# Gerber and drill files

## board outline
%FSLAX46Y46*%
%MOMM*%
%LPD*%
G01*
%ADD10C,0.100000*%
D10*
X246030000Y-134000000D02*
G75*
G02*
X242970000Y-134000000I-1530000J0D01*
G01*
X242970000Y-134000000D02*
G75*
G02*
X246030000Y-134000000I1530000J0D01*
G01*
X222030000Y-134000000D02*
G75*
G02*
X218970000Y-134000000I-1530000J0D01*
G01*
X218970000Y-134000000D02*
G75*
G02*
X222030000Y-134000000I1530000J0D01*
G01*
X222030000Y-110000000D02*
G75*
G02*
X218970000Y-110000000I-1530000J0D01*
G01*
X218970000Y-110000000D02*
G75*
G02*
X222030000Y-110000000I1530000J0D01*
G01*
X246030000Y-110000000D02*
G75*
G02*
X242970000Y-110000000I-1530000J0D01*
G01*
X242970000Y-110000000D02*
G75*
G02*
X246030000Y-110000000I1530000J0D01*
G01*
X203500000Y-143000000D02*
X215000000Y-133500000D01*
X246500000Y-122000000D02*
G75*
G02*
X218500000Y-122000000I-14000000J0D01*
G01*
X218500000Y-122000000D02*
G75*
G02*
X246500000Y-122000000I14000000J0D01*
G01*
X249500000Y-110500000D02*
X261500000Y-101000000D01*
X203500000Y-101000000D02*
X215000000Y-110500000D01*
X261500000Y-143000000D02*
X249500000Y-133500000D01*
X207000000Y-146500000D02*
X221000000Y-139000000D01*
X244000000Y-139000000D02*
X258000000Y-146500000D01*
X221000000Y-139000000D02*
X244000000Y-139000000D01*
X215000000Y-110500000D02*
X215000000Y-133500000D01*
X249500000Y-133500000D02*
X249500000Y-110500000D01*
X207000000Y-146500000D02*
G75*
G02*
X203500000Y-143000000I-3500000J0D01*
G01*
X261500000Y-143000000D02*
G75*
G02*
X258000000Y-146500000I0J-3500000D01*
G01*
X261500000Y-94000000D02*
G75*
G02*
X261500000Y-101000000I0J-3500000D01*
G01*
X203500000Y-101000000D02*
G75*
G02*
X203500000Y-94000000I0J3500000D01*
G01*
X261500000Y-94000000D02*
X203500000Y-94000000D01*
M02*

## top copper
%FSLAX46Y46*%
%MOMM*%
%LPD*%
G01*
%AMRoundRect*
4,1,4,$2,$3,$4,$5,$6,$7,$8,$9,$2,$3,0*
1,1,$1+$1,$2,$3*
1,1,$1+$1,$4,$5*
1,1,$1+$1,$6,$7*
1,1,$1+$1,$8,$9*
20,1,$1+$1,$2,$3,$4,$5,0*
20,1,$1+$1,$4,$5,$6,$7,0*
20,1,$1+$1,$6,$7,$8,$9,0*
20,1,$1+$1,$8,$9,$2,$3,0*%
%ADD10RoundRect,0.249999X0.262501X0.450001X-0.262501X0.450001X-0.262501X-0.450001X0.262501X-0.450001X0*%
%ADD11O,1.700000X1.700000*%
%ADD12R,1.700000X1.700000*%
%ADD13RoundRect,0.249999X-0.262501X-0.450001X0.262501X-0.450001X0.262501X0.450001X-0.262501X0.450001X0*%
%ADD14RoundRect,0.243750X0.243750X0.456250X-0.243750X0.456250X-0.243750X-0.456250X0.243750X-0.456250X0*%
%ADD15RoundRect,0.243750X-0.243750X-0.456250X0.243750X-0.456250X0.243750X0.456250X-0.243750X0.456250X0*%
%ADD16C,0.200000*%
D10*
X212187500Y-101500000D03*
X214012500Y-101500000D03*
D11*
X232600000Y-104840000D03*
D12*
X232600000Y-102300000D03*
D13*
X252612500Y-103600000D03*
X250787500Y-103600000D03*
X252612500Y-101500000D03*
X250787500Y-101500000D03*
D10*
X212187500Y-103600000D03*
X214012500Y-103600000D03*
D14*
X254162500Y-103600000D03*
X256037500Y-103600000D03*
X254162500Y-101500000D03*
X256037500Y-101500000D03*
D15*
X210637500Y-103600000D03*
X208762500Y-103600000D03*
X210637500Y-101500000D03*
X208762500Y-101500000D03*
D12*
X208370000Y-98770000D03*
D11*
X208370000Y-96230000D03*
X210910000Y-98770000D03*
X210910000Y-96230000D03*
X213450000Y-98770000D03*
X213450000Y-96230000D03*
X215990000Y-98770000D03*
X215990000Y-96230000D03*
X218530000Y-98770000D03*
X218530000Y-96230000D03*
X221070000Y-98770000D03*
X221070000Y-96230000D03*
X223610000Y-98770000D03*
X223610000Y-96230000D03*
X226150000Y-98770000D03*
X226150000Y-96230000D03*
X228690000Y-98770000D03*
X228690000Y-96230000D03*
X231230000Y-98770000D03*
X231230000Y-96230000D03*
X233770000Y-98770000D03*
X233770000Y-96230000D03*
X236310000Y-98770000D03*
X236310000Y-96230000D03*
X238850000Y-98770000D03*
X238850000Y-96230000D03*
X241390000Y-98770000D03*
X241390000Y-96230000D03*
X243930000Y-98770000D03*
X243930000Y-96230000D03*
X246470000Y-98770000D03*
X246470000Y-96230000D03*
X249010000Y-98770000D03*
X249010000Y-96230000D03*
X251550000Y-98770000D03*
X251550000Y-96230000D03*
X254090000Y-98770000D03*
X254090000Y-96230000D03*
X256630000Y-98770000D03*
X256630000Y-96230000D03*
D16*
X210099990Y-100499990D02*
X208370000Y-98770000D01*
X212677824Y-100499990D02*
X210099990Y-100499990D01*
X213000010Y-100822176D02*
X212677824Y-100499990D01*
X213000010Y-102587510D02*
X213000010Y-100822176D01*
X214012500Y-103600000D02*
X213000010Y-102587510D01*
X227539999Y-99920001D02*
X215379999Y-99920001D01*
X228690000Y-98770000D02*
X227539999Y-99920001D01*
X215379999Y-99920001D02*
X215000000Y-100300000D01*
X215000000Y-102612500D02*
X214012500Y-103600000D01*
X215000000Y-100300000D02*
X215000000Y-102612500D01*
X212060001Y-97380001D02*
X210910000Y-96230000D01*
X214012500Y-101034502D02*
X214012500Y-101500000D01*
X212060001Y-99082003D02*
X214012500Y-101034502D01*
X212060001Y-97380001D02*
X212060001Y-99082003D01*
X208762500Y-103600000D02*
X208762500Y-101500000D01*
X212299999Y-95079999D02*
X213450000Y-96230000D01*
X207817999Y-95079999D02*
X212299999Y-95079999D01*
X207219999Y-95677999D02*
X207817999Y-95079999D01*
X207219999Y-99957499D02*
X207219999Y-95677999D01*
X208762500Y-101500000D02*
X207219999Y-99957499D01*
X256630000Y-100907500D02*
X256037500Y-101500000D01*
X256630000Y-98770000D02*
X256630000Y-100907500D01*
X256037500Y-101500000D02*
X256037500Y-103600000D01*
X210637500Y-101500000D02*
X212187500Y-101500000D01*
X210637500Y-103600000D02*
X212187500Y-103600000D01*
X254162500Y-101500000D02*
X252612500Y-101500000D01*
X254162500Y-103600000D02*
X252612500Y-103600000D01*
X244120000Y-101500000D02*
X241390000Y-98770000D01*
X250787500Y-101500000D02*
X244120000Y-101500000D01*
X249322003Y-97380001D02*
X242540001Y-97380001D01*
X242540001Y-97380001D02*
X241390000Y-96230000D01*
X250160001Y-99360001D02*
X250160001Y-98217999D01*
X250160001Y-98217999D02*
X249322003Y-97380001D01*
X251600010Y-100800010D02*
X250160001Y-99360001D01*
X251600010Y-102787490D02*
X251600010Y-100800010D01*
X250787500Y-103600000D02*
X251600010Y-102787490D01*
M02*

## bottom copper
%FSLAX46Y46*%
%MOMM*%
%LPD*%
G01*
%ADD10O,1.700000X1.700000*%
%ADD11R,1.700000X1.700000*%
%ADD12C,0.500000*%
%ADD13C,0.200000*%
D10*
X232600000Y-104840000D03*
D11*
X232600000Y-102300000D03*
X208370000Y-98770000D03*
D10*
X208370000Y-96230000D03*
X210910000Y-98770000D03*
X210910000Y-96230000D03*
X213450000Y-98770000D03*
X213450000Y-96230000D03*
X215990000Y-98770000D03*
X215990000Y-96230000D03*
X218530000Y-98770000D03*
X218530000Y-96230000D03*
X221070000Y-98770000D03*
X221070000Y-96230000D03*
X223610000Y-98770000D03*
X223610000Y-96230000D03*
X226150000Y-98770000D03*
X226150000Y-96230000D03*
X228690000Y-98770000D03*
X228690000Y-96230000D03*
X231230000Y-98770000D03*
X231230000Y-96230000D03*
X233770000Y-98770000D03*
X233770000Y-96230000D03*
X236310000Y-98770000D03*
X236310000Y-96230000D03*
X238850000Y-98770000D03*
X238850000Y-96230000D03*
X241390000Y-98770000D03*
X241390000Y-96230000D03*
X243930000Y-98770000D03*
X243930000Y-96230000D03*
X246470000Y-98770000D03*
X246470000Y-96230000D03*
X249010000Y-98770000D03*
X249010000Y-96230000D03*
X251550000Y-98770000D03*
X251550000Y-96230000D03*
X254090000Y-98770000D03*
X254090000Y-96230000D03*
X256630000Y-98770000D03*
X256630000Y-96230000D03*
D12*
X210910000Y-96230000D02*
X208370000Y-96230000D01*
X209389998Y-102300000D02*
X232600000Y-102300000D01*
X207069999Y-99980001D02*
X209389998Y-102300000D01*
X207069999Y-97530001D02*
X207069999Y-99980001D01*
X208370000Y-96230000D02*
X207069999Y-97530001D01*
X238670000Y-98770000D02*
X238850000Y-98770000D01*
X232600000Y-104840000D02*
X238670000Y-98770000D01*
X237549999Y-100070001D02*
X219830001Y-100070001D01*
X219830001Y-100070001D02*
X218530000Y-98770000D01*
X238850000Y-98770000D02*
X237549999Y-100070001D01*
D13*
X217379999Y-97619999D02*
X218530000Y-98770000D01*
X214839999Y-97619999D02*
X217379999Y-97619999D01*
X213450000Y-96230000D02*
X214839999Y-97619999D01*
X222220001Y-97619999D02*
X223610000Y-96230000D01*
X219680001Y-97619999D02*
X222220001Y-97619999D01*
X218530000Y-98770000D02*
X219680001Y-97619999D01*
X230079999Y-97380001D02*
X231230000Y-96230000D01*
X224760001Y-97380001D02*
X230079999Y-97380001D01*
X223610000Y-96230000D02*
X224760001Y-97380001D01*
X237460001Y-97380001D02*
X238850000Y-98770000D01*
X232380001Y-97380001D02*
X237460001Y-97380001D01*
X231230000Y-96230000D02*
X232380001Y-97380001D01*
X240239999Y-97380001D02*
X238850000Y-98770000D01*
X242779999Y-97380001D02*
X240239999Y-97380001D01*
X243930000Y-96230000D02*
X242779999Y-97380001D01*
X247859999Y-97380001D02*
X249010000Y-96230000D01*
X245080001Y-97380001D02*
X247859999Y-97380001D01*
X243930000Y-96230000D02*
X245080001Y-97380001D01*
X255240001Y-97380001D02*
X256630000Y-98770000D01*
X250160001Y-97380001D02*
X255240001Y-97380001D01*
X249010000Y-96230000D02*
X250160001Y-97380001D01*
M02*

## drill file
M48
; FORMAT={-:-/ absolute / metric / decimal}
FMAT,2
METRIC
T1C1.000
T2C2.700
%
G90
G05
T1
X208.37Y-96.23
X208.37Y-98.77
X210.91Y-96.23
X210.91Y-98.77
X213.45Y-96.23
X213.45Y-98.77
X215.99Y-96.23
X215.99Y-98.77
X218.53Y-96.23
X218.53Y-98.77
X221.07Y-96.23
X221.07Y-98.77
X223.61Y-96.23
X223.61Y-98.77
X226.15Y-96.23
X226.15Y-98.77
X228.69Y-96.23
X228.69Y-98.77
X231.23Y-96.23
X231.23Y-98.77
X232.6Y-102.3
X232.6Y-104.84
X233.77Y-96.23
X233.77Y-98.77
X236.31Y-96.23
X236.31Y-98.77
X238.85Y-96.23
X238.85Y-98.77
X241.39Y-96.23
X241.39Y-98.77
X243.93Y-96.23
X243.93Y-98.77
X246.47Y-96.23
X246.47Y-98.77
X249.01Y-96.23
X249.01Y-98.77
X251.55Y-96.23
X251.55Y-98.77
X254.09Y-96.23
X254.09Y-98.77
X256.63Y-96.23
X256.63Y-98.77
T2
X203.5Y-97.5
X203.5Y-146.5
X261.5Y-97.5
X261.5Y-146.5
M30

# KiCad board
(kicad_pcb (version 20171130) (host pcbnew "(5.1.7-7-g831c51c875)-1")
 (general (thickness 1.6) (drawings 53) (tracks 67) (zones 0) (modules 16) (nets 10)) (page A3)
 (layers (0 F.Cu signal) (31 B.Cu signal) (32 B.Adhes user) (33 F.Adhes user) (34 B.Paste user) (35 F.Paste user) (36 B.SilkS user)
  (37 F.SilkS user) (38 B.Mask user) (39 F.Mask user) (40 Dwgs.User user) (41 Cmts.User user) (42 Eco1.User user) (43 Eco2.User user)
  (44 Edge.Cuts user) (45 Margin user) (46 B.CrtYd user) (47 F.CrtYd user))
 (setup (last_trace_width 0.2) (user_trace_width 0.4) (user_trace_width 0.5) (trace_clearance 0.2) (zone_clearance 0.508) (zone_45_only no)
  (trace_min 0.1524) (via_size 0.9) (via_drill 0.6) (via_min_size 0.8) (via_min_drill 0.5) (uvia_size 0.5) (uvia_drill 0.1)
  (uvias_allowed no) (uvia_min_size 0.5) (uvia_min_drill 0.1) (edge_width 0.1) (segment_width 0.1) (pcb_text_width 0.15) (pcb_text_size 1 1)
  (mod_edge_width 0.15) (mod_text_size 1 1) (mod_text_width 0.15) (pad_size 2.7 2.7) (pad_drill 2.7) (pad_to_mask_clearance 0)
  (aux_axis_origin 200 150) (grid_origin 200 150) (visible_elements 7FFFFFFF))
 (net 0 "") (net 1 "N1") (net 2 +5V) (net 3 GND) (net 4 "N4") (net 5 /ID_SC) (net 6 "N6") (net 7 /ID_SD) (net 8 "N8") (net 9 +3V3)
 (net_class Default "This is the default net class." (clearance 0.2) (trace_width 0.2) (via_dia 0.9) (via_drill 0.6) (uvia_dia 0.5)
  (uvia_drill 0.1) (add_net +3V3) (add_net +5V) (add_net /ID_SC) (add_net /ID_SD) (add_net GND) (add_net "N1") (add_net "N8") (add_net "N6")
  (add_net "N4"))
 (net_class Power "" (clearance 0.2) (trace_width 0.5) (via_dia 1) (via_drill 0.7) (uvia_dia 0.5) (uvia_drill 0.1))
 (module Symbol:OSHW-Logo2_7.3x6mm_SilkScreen (layer F.Cu) (at 251 138.3)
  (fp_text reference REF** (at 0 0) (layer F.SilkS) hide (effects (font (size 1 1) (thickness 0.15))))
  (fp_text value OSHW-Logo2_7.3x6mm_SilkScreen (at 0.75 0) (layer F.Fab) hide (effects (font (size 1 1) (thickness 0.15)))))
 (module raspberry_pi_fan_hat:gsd (layer F.Cu) (at 213.9 138.30663)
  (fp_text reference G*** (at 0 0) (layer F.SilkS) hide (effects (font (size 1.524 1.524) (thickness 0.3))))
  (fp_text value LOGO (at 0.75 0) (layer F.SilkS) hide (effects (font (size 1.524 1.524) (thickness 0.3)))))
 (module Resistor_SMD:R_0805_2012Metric (layer F.Cu) (at 213.1 101.5 180)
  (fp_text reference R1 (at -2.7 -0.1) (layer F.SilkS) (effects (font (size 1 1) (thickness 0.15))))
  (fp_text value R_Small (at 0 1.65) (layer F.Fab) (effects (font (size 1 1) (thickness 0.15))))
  (pad 2 smd roundrect (at 0.9125 0 180) (size 1.025 1.4) (layers F.Cu F.Paste F.Mask) (roundrect_rratio 0.2439014634146341) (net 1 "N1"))
  (pad 1 smd roundrect (at -0.9125 0 180) (size 1.025 1.4) (layers F.Cu F.Paste F.Mask) (roundrect_rratio 0.2439014634146341) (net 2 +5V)))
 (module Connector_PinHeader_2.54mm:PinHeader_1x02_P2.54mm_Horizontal (layer F.Cu) (at 232.6 102.3)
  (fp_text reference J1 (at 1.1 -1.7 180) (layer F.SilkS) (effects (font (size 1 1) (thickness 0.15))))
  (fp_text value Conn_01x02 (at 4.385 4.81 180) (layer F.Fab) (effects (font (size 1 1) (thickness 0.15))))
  (pad 2 thru_hole oval (at 0 2.54) (size 1.7 1.7) (drill 1) (layers *.Cu *.Mask) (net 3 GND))
  (pad 1 thru_hole rect (at 0 0) (size 1.7 1.7) (drill 1) (layers *.Cu *.Mask) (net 2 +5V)))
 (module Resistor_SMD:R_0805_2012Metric (layer F.Cu) (at 251.7 103.6)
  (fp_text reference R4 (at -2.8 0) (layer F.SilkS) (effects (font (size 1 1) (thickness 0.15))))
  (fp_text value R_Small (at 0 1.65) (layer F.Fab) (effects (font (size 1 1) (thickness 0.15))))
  (pad 2 smd roundrect (at 0.9125 0) (size 1.025 1.4) (layers F.Cu F.Paste F.Mask) (roundrect_rratio 0.2439014634146341) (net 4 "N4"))
  (pad 1 smd roundrect (at -0.9125 0) (size 1.025 1.4) (layers F.Cu F.Paste F.Mask) (roundrect_rratio 0.2439014634146341) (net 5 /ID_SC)))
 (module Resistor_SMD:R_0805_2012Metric (layer F.Cu) (at 251.7 101.5)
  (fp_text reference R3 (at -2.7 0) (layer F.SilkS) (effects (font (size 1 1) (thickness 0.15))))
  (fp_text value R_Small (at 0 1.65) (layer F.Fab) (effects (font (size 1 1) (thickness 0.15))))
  (pad 2 smd roundrect (at 0.9125 0) (size 1.025 1.4) (layers F.Cu F.Paste F.Mask) (roundrect_rratio 0.2439014634146341) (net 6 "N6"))
  (pad 1 smd roundrect (at -0.9125 0) (size 1.025 1.4) (layers F.Cu F.Paste F.Mask) (roundrect_rratio 0.2439014634146341) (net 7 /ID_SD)))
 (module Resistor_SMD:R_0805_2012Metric (layer F.Cu) (at 213.1 103.6 180)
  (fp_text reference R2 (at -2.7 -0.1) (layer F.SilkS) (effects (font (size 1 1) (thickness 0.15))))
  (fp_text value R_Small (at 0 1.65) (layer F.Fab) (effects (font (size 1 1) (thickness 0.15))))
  (pad 2 smd roundrect (at 0.9125 0 180) (size 1.025 1.4) (layers F.Cu F.Paste F.Mask) (roundrect_rratio 0.2439014634146341) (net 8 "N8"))
  (pad 1 smd roundrect (at -0.9125 0 180) (size 1.025 1.4) (layers F.Cu F.Paste F.Mask) (roundrect_rratio 0.2439014634146341) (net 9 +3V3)))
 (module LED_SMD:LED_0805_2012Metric (layer F.Cu) (at 255.1 103.6 180)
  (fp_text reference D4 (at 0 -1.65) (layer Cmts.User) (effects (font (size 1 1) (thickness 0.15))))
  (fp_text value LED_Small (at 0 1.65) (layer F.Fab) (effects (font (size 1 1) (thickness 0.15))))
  (pad 2 smd roundrect (at 0.9375 0 180) (size 0.975 1.4) (layers F.Cu F.Paste F.Mask) (roundrect_rratio 0.25) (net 4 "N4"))
  (pad 1 smd roundrect (at -0.9375 0 180) (size 0.975 1.4) (layers F.Cu F.Paste F.Mask) (roundrect_rratio 0.25) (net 3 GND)))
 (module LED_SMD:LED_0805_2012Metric (layer F.Cu) (at 255.1 101.5 180)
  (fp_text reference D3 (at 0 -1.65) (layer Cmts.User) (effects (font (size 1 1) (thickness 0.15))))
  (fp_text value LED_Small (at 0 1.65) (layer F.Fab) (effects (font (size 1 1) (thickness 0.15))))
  (pad 2 smd roundrect (at 0.9375 0 180) (size 0.975 1.4) (layers F.Cu F.Paste F.Mask) (roundrect_rratio 0.25) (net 6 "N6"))
  (pad 1 smd roundrect (at -0.9375 0 180) (size 0.975 1.4) (layers F.Cu F.Paste F.Mask) (roundrect_rratio 0.25) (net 3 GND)))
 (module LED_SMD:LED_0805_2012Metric (layer F.Cu) (at 209.7 103.6)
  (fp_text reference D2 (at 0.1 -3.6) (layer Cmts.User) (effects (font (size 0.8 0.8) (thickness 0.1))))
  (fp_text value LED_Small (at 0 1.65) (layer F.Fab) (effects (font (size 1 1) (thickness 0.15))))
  (pad 2 smd roundrect (at 0.9375 0) (size 0.975 1.4) (layers F.Cu F.Paste F.Mask) (roundrect_rratio 0.25) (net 8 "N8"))
  (pad 1 smd roundrect (at -0.9375 0) (size 0.975 1.4) (layers F.Cu F.Paste F.Mask) (roundrect_rratio 0.25) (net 3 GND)))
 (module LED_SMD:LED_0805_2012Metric (layer F.Cu) (at 209.7 101.5)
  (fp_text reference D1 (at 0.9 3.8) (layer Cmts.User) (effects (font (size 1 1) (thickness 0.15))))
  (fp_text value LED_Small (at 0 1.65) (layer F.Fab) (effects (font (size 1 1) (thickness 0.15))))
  (pad 2 smd roundrect (at 0.9375 0) (size 0.975 1.4) (layers F.Cu F.Paste F.Mask) (roundrect_rratio 0.25) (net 1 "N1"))
  (pad 1 smd roundrect (at -0.9375 0) (size 0.975 1.4) (layers F.Cu F.Paste F.Mask) (roundrect_rratio 0.25) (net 3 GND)))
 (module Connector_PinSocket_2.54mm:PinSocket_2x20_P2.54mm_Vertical (layer B.Cu) (at 208.37 98.77 270)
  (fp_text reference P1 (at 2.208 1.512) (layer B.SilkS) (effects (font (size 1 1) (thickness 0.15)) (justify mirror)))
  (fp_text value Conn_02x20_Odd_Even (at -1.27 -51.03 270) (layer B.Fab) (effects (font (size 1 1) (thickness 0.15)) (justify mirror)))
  (pad 1 thru_hole rect (at 0 0 270) (size 1.7 1.7) (drill 1) (layers *.Cu *.Mask) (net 9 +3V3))
  (pad 2 thru_hole oval (at -2.54 0 270) (size 1.7 1.7) (drill 1) (layers *.Cu *.Mask) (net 2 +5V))
  (pad 3 thru_hole oval (at 0 -2.54 270) (size 1.7 1.7) (drill 1) (layers *.Cu *.Mask))
  (pad 4 thru_hole oval (at -2.54 -2.54 270) (size 1.7 1.7) (drill 1) (layers *.Cu *.Mask) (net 2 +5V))
  (pad 5 thru_hole oval (at 0 -5.08 270) (size 1.7 1.7) (drill 1) (layers *.Cu *.Mask))
  (pad 6 thru_hole oval (at -2.54 -5.08 270) (size 1.7 1.7) (drill 1) (layers *.Cu *.Mask) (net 3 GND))
  (pad 7 thru_hole oval (at 0 -7.62 270) (size 1.7 1.7) (drill 1) (layers *.Cu *.Mask))
  (pad 8 thru_hole oval (at -2.54 -7.62 270) (size 1.7 1.7) (drill 1) (layers *.Cu *.Mask))
  (pad 9 thru_hole oval (at 0 -10.16 270) (size 1.7 1.7) (drill 1) (layers *.Cu *.Mask) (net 3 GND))
  (pad 10 thru_hole oval (at -2.54 -10.16 270) (size 1.7 1.7) (drill 1) (layers *.Cu *.Mask))
  (pad 11 thru_hole oval (at 0 -12.7 270) (size 1.7 1.7) (drill 1) (layers *.Cu *.Mask))
  (pad 12 thru_hole oval (at -2.54 -12.7 270) (size 1.7 1.7) (drill 1) (layers *.Cu *.Mask))
  (pad 13 thru_hole oval (at 0 -15.24 270) (size 1.7 1.7) (drill 1) (layers *.Cu *.Mask))
  (pad 14 thru_hole oval (at -2.54 -15.24 270) (size 1.7 1.7) (drill 1) (layers *.Cu *.Mask) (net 3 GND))
  (pad 15 thru_hole oval (at 0 -17.78 270) (size 1.7 1.7) (drill 1) (layers *.Cu *.Mask))
  (pad 16 thru_hole oval (at -2.54 -17.78 270) (size 1.7 1.7) (drill 1) (layers *.Cu *.Mask))
  (pad 17 thru_hole oval (at 0 -20.32 270) (size 1.7 1.7) (drill 1) (layers *.Cu *.Mask) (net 9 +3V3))
  (pad 18 thru_hole oval (at -2.54 -20.32 270) (size 1.7 1.7) (drill 1) (layers *.Cu *.Mask))
  (pad 19 thru_hole oval (at 0 -22.86 270) (size 1.7 1.7) (drill 1) (layers *.Cu *.Mask))
  (pad 20 thru_hole oval (at -2.54 -22.86 270) (size 1.7 1.7) (drill 1) (layers *.Cu *.Mask) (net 3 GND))
  (pad 21 thru_hole oval (at 0 -25.4 270) (size 1.7 1.7) (drill 1) (layers *.Cu *.Mask))
  (pad 22 thru_hole oval (at -2.54 -25.4 270) (size 1.7 1.7) (drill 1) (layers *.Cu *.Mask))
  (pad 23 thru_hole oval (at 0 -27.94 270) (size 1.7 1.7) (drill 1) (layers *.Cu *.Mask))
  (pad 24 thru_hole oval (at -2.54 -27.94 270) (size 1.7 1.7) (drill 1) (layers *.Cu *.Mask))
  (pad 25 thru_hole oval (at 0 -30.48 270) (size 1.7 1.7) (drill 1) (layers *.Cu *.Mask) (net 3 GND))
  (pad 26 thru_hole oval (at -2.54 -30.48 270) (size 1.7 1.7) (drill 1) (layers *.Cu *.Mask))
  (pad 27 thru_hole oval (at 0 -33.02 270) (size 1.7 1.7) (drill 1) (layers *.Cu *.Mask) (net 7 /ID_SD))
  (pad 28 thru_hole oval (at -2.54 -33.02 270) (size 1.7 1.7) (drill 1) (layers *.Cu *.Mask) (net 5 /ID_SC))
  (pad 29 thru_hole oval (at 0 -35.56 270) (size 1.7 1.7) (drill 1) (layers *.Cu *.Mask))
  (pad 30 thru_hole oval (at -2.54 -35.56 270) (size 1.7 1.7) (drill 1) (layers *.Cu *.Mask) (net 3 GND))
  (pad 31 thru_hole oval (at 0 -38.1 270) (size 1.7 1.7) (drill 1) (layers *.Cu *.Mask))
  (pad 32 thru_hole oval (at -2.54 -38.1 270) (size 1.7 1.7) (drill 1) (layers *.Cu *.Mask))
  (pad 33 thru_hole oval (at 0 -40.64 270) (size 1.7 1.7) (drill 1) (layers *.Cu *.Mask))
  (pad 34 thru_hole oval (at -2.54 -40.64 270) (size 1.7 1.7) (drill 1) (layers *.Cu *.Mask) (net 3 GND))
  (pad 35 thru_hole oval (at 0 -43.18 270) (size 1.7 1.7) (drill 1) (layers *.Cu *.Mask))
  (pad 36 thru_hole oval (at -2.54 -43.18 270) (size 1.7 1.7) (drill 1) (layers *.Cu *.Mask))
  (pad 37 thru_hole oval (at 0 -45.72 270) (size 1.7 1.7) (drill 1) (layers *.Cu *.Mask))
  (pad 38 thru_hole oval (at -2.54 -45.72 270) (size 1.7 1.7) (drill 1) (layers *.Cu *.Mask))
  (pad 39 thru_hole oval (at 0 -48.26 270) (size 1.7 1.7) (drill 1) (layers *.Cu *.Mask) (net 3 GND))
  (pad 40 thru_hole oval (at -2.54 -48.26 270) (size 1.7 1.7) (drill 1) (layers *.Cu *.Mask)))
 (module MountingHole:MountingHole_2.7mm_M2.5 (layer F.Cu) (at 261.5 146.5)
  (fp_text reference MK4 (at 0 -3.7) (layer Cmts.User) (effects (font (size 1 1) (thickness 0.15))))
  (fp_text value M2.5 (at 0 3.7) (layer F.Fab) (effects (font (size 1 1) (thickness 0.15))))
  (pad 1 np_thru_hole circle (at 0 0) (size 2.7 2.7) (drill 2.7) (layers *.Cu *.Mask)))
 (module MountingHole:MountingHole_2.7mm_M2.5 (layer F.Cu) (at 203.5 146.5)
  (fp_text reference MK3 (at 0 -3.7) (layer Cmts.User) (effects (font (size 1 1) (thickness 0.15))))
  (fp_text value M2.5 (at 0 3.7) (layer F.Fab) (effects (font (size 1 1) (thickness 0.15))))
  (pad 1 np_thru_hole circle (at 0 0) (size 2.7 2.7) (drill 2.7) (layers *.Cu *.Mask)))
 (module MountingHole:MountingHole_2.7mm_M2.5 (layer F.Cu) (at 261.5 97.5 180)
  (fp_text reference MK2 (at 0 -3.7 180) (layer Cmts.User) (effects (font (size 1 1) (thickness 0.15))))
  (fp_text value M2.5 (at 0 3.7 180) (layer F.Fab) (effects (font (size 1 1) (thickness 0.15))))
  (pad 1 np_thru_hole circle (at 0 0 180) (size 2.7 2.7) (drill 2.7) (layers *.Cu *.Mask)))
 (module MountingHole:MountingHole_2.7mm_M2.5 (layer F.Cu) (at 203.5 97.5 180)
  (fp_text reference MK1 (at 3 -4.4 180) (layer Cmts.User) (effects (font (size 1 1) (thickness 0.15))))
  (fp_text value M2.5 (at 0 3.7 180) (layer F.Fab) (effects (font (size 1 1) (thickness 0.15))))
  (pad "" np_thru_hole circle (at 0 0 180) (size 2.7 2.7) (drill 2.7) (layers *.Cu *.Mask)))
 (gr_circle (center 244.5 134) (end 246.03 134) (layer Edge.Cuts) (width 0.1))
 (gr_circle (center 220.5 134) (end 222.03 134) (layer Edge.Cuts) (width 0.1))
 (gr_circle (center 220.5 110) (end 222.03 110) (layer Edge.Cuts) (width 0.1))
 (gr_circle (center 244.5 110) (end 246.03 110) (layer Edge.Cuts) (width 0.1))
 (gr_line (start 203.5 143) (end 215 133.5) (layer Edge.Cuts) (width 0.1))
 (gr_circle (center 232.5 122) (end 246.5 122) (layer Edge.Cuts) (width 0.1))
 (gr_line (start 249.5 110.5) (end 261.5 101) (layer Edge.Cuts) (width 0.1))
 (gr_line (start 203.5 101) (end 215 110.5) (layer Edge.Cuts) (width 0.1))
 (gr_line (start 261.5 143) (end 249.5 133.5) (layer Edge.Cuts) (width 0.1))
 (gr_line (start 207 146.5) (end 221 139) (layer Edge.Cuts) (width 0.1))
 (gr_line (start 244 139) (end 258 146.5) (layer Edge.Cuts) (width 0.1))
 (gr_line (start 221 139) (end 244 139) (layer Edge.Cuts) (width 0.1))
 (gr_line (start 215 110.5) (end 215 133.5) (layer Edge.Cuts) (width 0.1))
 (gr_line (start 249.5 133.5) (end 249.5 110.5) (layer Edge.Cuts) (width 0.1))
 (gr_arc (start 203.5 146.5) (end 203.5 143) (angle -270) (layer Edge.Cuts) (width 0.1))
 (gr_arc (start 261.5 146.5) (end 258 146.5) (angle -270) (layer Edge.Cuts) (width 0.1))
 (gr_arc (start 261.5 97.5) (end 261.5 101) (angle -180) (layer Edge.Cuts) (width 0.1))
 (gr_arc (start 203.5 97.5) (end 203.5 94) (angle -180) (layer Edge.Cuts) (width 0.1))
 (gr_line (start 261.5 94) (end 203.5 94) (layer Edge.Cuts) (width 0.1))
 (segment (start 210.09999 100.49999) (end 208.37 98.77) (width 0.2) (layer F.Cu) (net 9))
 (segment (start 212.677824 100.49999) (end 210.09999 100.49999) (width 0.2) (layer F.Cu) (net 9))
 (segment (start 213.00001 100.822176) (end 212.677824 100.49999) (width 0.2) (layer F.Cu) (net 9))
 (segment (start 213.00001 102.58751) (end 213.00001 100.822176) (width 0.2) (layer F.Cu) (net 9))
 (segment (start 214.0125 103.6) (end 213.00001 102.58751) (width 0.2) (layer F.Cu) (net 9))
 (segment (start 227.539999 99.920001) (end 215.379999 99.920001) (width 0.2) (layer F.Cu) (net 9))
 (segment (start 228.69 98.77) (end 227.539999 99.920001) (width 0.2) (layer F.Cu) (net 9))
 (segment (start 215.379999 99.920001) (end 215 100.3) (width 0.2) (layer F.Cu) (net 9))
 (segment (start 215 102.6125) (end 214.0125 103.6) (width 0.2) (layer F.Cu) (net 9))
 (segment (start 215 100.3) (end 215 102.6125) (width 0.2) (layer F.Cu) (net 9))
 (segment (start 210.91 96.23) (end 208.37 96.23) (width 0.5) (layer B.Cu) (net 2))
 (segment (start 209.389998 102.3) (end 232.6 102.3) (width 0.5) (layer B.Cu) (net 2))
 (segment (start 207.069999 99.980001) (end 209.389998 102.3) (width 0.5) (layer B.Cu) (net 2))
 (segment (start 207.069999 97.530001) (end 207.069999 99.980001) (width 0.5) (layer B.Cu) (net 2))
 (segment (start 208.37 96.23) (end 207.069999 97.530001) (width 0.5) (layer B.Cu) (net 2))
 (segment (start 212.060001 97.380001) (end 210.91 96.23) (width 0.2) (layer F.Cu) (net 2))
 (segment (start 214.0125 101.034502) (end 214.0125 101.5) (width 0.2) (layer F.Cu) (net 2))
 (segment (start 212.060001 99.082003) (end 214.0125 101.034502) (width 0.2) (layer F.Cu) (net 2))
 (segment (start 212.060001 97.380001) (end 212.060001 99.082003) (width 0.2) (layer F.Cu) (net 2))
 (segment (start 238.67 98.77) (end 238.85 98.77) (width 0.5) (layer B.Cu) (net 3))
 (segment (start 232.6 104.84) (end 238.67 98.77) (width 0.5) (layer B.Cu) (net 3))
 (segment (start 237.549999 100.070001) (end 219.830001 100.070001) (width 0.5) (layer B.Cu) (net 3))
 (segment (start 219.830001 100.070001) (end 218.53 98.77) (width 0.5) (layer B.Cu) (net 3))
 (segment (start 238.85 98.77) (end 237.549999 100.070001) (width 0.5) (layer B.Cu) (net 3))
 (segment (start 208.7625 103.6) (end 208.7625 101.5) (width 0.2) (layer F.Cu) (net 3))
 (segment (start 212.299999 95.079999) (end 213.45 96.23) (width 0.2) (layer F.Cu) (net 3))
 (segment (start 207.817999 95.079999) (end 212.299999 95.079999) (width 0.2) (layer F.Cu) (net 3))
 (segment (start 207.219999 95.677999) (end 207.817999 95.079999) (width 0.2) (layer F.Cu) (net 3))
 (segment (start 207.219999 99.957499) (end 207.219999 95.677999) (width 0.2) (layer F.Cu) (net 3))
 (segment (start 208.7625 101.5) (end 207.219999 99.957499) (width 0.2) (layer F.Cu) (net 3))
 (segment (start 256.63 100.9075) (end 256.0375 101.5) (width 0.2) (layer F.Cu) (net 3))
 (segment (start 256.63 98.77) (end 256.63 100.9075) (width 0.2) (layer F.Cu) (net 3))
 (segment (start 256.0375 101.5) (end 256.0375 103.6) (width 0.2) (layer F.Cu) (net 3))
 (segment (start 217.379999 97.619999) (end 218.53 98.77) (width 0.2) (layer B.Cu) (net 3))
 (segment (start 214.839999 97.619999) (end 217.379999 97.619999) (width 0.2) (layer B.Cu) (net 3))
 (segment (start 213.45 96.23) (end 214.839999 97.619999) (width 0.2) (layer B.Cu) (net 3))
 (segment (start 222.220001 97.619999) (end 223.61 96.23) (width 0.2) (layer B.Cu) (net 3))
 (segment (start 219.680001 97.619999) (end 222.220001 97.619999) (width 0.2) (layer B.Cu) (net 3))
 (segment (start 218.53 98.77) (end 219.680001 97.619999) (width 0.2) (layer B.Cu) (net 3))
 (segment (start 230.079999 97.380001) (end 231.23 96.23) (width 0.2) (layer B.Cu) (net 3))
 (segment (start 224.760001 97.380001) (end 230.079999 97.380001) (width 0.2) (layer B.Cu) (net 3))
 (segment (start 223.61 96.23) (end 224.760001 97.380001) (width 0.2) (layer B.Cu) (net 3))
 (segment (start 237.460001 97.380001) (end 238.85 98.77) (width 0.2) (layer B.Cu) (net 3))
 (segment (start 232.380001 97.380001) (end 237.460001 97.380001) (width 0.2) (layer B.Cu) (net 3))
 (segment (start 231.23 96.23) (end 232.380001 97.380001) (width 0.2) (layer B.Cu) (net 3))
 (segment (start 240.239999 97.380001) (end 238.85 98.77) (width 0.2) (layer B.Cu) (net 3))
 (segment (start 242.779999 97.380001) (end 240.239999 97.380001) (width 0.2) (layer B.Cu) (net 3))
 (segment (start 243.93 96.23) (end 242.779999 97.380001) (width 0.2) (layer B.Cu) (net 3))
 (segment (start 247.859999 97.380001) (end 249.01 96.23) (width 0.2) (layer B.Cu) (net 3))
 (segment (start 245.080001 97.380001) (end 247.859999 97.380001) (width 0.2) (layer B.Cu) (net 3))
 (segment (start 243.93 96.23) (end 245.080001 97.380001) (width 0.2) (layer B.Cu) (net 3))
 (segment (start 255.240001 97.380001) (end 256.63 98.77) (width 0.2) (layer B.Cu) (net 3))
 (segment (start 250.160001 97.380001) (end 255.240001 97.380001) (width 0.2) (layer B.Cu) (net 3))
 (segment (start 249.01 96.23) (end 250.160001 97.380001) (width 0.2) (layer B.Cu) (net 3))
 (segment (start 210.6375 101.5) (end 212.1875 101.5) (width 0.2) (layer F.Cu) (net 1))
 (segment (start 210.6375 103.6) (end 212.1875 103.6) (width 0.2) (layer F.Cu) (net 8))
 (segment (start 254.1625 101.5) (end 252.6125 101.5) (width 0.2) (layer F.Cu) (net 6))
 (segment (start 254.1625 103.6) (end 252.6125 103.6) (width 0.2) (layer F.Cu) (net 4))
 (segment (start 244.12 101.5) (end 241.39 98.77) (width 0.2) (layer F.Cu) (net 7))
 (segment (start 250.7875 101.5) (end 244.12 101.5) (width 0.2) (layer F.Cu) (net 7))
 (segment (start 249.322003 97.380001) (end 242.540001 97.380001) (width 0.2) (layer F.Cu) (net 5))
 (segment (start 242.540001 97.380001) (end 241.39 96.23) (width 0.2) (layer F.Cu) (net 5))
 (segment (start 250.160001 99.360001) (end 250.160001 98.217999) (width 0.2) (layer F.Cu) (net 5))
 (segment (start 250.160001 98.217999) (end 249.322003 97.380001) (width 0.2) (layer F.Cu) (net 5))
 (segment (start 251.60001 100.80001) (end 250.160001 99.360001) (width 0.2) (layer F.Cu) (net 5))
 (segment (start 251.60001 102.78749) (end 251.60001 100.80001) (width 0.2) (layer F.Cu) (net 5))
 (segment (start 250.7875 103.6) (end 251.60001 102.78749) (width 0.2) (layer F.Cu) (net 5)))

